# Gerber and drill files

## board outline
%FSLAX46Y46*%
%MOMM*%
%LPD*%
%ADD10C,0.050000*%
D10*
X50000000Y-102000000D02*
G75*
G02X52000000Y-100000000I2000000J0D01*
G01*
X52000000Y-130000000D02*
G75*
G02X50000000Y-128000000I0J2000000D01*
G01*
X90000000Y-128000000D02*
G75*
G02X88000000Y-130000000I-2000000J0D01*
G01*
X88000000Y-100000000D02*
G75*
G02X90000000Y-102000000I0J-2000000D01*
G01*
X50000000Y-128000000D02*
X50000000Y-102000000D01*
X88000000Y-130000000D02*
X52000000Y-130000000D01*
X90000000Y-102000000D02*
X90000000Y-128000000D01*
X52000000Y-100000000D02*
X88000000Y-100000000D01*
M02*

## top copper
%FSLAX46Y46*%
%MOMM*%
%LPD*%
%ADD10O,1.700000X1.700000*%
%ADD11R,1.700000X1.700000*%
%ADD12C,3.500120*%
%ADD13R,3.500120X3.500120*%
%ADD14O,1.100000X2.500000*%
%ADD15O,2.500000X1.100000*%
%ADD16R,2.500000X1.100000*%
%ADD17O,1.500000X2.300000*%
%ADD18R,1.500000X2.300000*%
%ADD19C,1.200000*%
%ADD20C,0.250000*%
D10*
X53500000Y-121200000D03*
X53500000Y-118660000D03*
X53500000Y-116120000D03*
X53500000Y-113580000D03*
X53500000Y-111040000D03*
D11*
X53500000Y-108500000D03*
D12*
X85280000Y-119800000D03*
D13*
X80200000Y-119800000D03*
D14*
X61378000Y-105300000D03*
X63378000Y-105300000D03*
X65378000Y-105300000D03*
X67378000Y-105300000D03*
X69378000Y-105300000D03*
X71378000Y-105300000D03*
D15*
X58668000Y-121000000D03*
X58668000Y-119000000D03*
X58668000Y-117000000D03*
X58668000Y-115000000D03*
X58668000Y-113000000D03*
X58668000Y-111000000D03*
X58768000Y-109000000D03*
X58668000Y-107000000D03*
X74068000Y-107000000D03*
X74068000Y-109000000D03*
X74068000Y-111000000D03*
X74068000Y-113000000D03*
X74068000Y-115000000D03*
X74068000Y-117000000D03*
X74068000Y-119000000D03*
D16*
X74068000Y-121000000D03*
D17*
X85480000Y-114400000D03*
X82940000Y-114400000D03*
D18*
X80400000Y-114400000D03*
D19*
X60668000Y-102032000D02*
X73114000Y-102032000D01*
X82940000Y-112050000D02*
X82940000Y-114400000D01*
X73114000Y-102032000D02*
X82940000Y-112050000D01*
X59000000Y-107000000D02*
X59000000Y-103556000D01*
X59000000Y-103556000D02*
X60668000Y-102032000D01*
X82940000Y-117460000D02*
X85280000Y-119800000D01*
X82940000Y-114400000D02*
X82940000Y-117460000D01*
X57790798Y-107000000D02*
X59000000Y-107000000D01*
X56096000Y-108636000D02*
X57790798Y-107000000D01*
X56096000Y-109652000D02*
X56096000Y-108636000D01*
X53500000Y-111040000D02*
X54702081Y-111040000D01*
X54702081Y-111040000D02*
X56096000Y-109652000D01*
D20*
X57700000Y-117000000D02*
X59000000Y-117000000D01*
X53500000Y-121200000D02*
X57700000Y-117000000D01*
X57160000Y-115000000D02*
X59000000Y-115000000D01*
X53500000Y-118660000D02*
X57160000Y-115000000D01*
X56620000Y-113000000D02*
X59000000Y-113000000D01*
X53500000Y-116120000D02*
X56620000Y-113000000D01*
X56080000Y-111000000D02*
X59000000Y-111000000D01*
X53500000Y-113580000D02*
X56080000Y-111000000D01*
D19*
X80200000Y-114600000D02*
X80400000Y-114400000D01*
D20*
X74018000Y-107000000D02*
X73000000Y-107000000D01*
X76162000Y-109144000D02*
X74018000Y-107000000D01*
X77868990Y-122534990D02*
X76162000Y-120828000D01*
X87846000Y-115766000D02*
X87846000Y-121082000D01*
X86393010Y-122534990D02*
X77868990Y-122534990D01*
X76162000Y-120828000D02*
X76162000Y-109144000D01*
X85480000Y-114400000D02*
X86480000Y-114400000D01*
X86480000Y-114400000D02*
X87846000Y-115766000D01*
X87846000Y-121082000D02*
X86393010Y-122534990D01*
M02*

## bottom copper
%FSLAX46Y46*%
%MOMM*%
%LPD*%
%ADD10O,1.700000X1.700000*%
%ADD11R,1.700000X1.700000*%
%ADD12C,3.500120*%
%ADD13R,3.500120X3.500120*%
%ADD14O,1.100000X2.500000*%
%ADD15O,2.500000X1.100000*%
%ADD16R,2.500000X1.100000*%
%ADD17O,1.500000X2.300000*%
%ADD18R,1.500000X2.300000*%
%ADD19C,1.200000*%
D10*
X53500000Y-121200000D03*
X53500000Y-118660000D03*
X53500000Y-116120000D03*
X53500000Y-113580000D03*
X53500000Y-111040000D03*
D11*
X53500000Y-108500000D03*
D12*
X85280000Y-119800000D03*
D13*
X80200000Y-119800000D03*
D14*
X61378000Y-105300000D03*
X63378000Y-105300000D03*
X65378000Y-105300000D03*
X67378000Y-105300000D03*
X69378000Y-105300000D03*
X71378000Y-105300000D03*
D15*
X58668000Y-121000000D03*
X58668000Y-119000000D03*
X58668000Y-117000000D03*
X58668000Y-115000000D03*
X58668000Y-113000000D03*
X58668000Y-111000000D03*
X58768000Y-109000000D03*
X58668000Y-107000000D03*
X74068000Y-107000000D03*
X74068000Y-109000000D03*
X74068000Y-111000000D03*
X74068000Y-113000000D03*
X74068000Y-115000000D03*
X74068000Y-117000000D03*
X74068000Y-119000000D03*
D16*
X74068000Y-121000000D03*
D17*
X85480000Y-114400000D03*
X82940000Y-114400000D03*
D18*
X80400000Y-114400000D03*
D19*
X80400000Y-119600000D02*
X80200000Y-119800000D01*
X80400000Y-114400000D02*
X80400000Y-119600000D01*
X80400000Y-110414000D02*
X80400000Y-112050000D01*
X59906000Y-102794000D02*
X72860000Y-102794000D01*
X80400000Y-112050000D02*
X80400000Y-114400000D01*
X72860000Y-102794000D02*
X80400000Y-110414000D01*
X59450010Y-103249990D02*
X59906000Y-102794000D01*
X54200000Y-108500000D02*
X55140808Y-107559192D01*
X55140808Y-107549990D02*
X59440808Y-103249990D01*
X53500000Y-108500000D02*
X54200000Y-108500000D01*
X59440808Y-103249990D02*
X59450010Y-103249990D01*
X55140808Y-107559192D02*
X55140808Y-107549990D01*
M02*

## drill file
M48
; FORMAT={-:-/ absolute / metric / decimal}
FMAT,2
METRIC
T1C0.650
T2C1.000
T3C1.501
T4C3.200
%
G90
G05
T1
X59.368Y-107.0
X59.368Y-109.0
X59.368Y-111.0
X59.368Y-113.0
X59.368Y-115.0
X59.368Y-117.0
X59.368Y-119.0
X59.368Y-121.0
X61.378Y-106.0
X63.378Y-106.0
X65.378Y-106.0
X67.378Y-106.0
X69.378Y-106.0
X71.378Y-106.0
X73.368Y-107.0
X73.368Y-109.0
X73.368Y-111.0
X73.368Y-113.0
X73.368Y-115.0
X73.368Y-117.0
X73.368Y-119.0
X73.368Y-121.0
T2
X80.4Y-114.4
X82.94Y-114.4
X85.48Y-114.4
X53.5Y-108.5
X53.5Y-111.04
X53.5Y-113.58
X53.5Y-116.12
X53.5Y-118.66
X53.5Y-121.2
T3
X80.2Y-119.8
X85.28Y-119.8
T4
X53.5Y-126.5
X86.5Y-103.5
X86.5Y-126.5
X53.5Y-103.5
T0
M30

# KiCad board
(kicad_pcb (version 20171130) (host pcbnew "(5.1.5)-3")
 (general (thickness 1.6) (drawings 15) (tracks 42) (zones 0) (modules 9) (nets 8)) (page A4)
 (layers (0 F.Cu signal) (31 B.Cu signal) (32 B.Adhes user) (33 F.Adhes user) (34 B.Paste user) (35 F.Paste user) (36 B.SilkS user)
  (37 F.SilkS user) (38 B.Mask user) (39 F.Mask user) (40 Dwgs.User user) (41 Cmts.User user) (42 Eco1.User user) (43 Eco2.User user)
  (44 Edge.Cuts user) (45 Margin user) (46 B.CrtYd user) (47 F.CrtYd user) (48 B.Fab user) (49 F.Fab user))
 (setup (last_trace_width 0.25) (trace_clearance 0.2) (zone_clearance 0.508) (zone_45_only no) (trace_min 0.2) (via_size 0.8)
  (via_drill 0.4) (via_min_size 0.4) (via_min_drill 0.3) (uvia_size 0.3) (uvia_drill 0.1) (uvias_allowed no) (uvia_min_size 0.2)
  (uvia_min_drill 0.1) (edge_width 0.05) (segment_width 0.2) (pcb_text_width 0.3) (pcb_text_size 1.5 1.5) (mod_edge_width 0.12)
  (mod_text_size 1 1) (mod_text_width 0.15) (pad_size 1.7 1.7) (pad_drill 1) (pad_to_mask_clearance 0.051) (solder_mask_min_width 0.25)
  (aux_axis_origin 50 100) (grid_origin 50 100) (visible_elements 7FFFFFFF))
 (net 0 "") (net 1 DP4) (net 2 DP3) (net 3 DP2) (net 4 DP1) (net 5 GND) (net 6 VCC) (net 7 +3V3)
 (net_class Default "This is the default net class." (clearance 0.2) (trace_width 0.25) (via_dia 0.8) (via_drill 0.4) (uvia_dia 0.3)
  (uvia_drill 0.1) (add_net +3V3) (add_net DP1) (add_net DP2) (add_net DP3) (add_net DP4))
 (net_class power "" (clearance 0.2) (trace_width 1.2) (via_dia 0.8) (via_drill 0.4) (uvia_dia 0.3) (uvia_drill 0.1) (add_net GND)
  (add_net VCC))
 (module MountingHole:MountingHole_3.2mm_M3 (layer F.Cu) (at 53.5 103.5)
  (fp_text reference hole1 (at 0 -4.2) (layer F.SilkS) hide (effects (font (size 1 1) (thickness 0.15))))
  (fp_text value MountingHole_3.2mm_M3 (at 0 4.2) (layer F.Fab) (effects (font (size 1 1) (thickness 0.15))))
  (pad 1 np_thru_hole circle (at 0 0) (size 3.2 3.2) (drill 3.2) (layers *.Cu *.Mask)))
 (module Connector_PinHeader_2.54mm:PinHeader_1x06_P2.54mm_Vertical (layer F.Cu) (at 53.5 108.5)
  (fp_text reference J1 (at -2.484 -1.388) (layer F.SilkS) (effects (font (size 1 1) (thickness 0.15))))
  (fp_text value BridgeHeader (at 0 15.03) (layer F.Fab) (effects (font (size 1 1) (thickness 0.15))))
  (pad 6 thru_hole oval (at 0 12.7) (size 1.7 1.7) (drill 1) (layers *.Cu *.Mask) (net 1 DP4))
  (pad 5 thru_hole oval (at 0 10.16) (size 1.7 1.7) (drill 1) (layers *.Cu *.Mask) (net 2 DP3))
  (pad 4 thru_hole oval (at 0 7.62) (size 1.7 1.7) (drill 1) (layers *.Cu *.Mask) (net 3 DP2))
  (pad 3 thru_hole oval (at 0 5.08) (size 1.7 1.7) (drill 1) (layers *.Cu *.Mask) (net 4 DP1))
  (pad 2 thru_hole oval (at 0 2.54) (size 1.7 1.7) (drill 1) (layers *.Cu *.Mask) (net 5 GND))
  (pad 1 thru_hole rect (at 0 0) (size 1.7 1.7) (drill 1) (layers *.Cu *.Mask) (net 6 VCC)))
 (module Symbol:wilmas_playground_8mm (layer F.Cu) (at 79.464 125.908)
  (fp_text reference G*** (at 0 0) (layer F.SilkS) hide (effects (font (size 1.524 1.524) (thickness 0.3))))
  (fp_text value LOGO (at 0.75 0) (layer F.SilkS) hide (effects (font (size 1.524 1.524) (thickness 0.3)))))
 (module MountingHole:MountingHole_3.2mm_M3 (layer F.Cu) (at 86.5 126.5)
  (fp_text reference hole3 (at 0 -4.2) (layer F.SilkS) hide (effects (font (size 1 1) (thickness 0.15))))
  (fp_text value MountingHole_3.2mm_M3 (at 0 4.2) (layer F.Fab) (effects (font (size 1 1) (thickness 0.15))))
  (pad 1 np_thru_hole circle (at 0 0) (size 3.2 3.2) (drill 3.2) (layers *.Cu *.Mask)))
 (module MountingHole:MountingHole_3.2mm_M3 (layer F.Cu) (at 86.5 103.5)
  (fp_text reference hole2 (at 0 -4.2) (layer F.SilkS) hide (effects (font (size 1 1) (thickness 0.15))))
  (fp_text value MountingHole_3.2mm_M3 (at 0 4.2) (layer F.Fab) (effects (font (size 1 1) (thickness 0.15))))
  (pad 1 np_thru_hole circle (at 0 0) (size 3.2 3.2) (drill 3.2) (layers *.Cu *.Mask)))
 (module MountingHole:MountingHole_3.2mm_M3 (layer F.Cu) (at 53.5 126.5)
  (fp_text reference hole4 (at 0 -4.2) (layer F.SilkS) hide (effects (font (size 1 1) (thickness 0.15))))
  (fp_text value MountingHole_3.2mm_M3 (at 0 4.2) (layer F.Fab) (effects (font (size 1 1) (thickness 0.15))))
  (pad 1 np_thru_hole circle (at 0 0) (size 3.2 3.2) (drill 3.2) (layers *.Cu *.Mask)))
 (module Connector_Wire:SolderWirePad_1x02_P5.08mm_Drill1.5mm (layer F.Cu) (at 80.2 119.8)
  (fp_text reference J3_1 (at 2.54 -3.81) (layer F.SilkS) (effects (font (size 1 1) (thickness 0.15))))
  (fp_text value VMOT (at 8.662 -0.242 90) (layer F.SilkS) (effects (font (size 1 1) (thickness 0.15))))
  (pad 2 thru_hole circle (at 5.08 0) (size 3.50012 3.50012) (drill 1.50114) (layers *.Cu *.Mask) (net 5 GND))
  (pad 1 thru_hole rect (at 0 0) (size 3.50012 3.50012) (drill 1.50114) (layers *.Cu *.Mask) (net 6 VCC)))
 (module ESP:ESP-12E (layer F.Cu) (at 73.368 121 180)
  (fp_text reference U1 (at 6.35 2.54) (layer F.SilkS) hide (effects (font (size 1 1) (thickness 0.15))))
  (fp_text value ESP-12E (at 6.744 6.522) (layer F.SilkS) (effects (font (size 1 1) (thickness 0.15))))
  (pad 22 thru_hole oval (at 11.99 15 270) (size 2.5 1.1) (drill 0.65 (offset -0.7 0)) (layers *.Cu *.Mask F.SilkS))
  (pad 21 thru_hole oval (at 9.99 15 270) (size 2.5 1.1) (drill 0.65 (offset -0.7 0)) (layers *.Cu *.Mask F.SilkS))
  (pad 20 thru_hole oval (at 7.99 15 270) (size 2.5 1.1) (drill 0.65 (offset -0.7 0)) (layers *.Cu *.Mask F.SilkS))
  (pad 19 thru_hole oval (at 5.99 15 270) (size 2.5 1.1) (drill 0.65 (offset -0.7 0)) (layers *.Cu *.Mask F.SilkS))
  (pad 18 thru_hole oval (at 3.99 15 270) (size 2.5 1.1) (drill 0.65 (offset -0.7 0)) (layers *.Cu *.Mask F.SilkS))
  (pad 17 thru_hole oval (at 1.99 15 270) (size 2.5 1.1) (drill 0.65 (offset -0.7 0)) (layers *.Cu *.Mask F.SilkS))
  (pad 16 thru_hole oval (at 14 0 180) (size 2.5 1.1) (drill 0.65 (offset 0.7 0)) (layers *.Cu *.Mask F.SilkS))
  (pad 15 thru_hole oval (at 14 2 180) (size 2.5 1.1) (drill 0.65 (offset 0.7 0)) (layers *.Cu *.Mask F.SilkS))
  (pad 14 thru_hole oval (at 14 4 180) (size 2.5 1.1) (drill 0.65 (offset 0.7 0)) (layers *.Cu *.Mask F.SilkS) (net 1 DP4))
  (pad 13 thru_hole oval (at 14 6 180) (size 2.5 1.1) (drill 0.65 (offset 0.7 0)) (layers *.Cu *.Mask F.SilkS) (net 2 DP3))
  (pad 12 thru_hole oval (at 14 8 180) (size 2.5 1.1) (drill 0.65 (offset 0.7 0)) (layers *.Cu *.Mask F.SilkS) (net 3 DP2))
  (pad 11 thru_hole oval (at 14 10 180) (size 2.5 1.1) (drill 0.65 (offset 0.7 0)) (layers *.Cu *.Mask F.SilkS) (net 4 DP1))
  (pad 10 thru_hole oval (at 14 12 180) (size 2.5 1.1) (drill 0.65 (offset 0.6 0)) (layers *.Cu *.Mask F.SilkS))
  (pad 9 thru_hole oval (at 14 14 180) (size 2.5 1.1) (drill 0.65 (offset 0.7 0)) (layers *.Cu *.Mask F.SilkS) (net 5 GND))
  (pad 8 thru_hole oval (at 0 14 180) (size 2.5 1.1) (drill 0.65 (offset -0.7 0)) (layers *.Cu *.Mask F.SilkS) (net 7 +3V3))
  (pad 7 thru_hole oval (at 0 12 180) (size 2.5 1.1) (drill 0.65 (offset -0.7 0)) (layers *.Cu *.Mask F.SilkS))
  (pad 6 thru_hole oval (at 0 10 180) (size 2.5 1.1) (drill 0.65 (offset -0.7 0)) (layers *.Cu *.Mask F.SilkS))
  (pad 5 thru_hole oval (at 0 8 180) (size 2.5 1.1) (drill 0.65 (offset -0.7 0)) (layers *.Cu *.Mask F.SilkS))
  (pad 4 thru_hole oval (at 0 6 180) (size 2.5 1.1) (drill 0.65 (offset -0.7 0)) (layers *.Cu *.Mask F.SilkS))
  (pad 3 thru_hole oval (at 0 4 180) (size 2.5 1.1) (drill 0.65 (offset -0.7 0)) (layers *.Cu *.Mask F.SilkS))
  (pad 2 thru_hole oval (at 0 2 180) (size 2.5 1.1) (drill 0.65 (offset -0.7 0)) (layers *.Cu *.Mask F.SilkS))
  (pad 1 thru_hole rect (at 0 0 180) (size 2.5 1.1) (drill 0.65 (offset -0.7 0)) (layers *.Cu *.Mask F.SilkS)))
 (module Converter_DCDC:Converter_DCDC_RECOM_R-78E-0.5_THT (layer F.Cu) (at 80.4 114.4)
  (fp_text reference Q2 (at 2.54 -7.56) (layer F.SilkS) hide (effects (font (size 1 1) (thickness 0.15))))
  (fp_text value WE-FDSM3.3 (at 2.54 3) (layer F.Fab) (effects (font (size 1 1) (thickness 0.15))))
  (pad 3 thru_hole oval (at 5.08 0) (size 1.5 2.3) (drill 1) (layers *.Cu *.Mask) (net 7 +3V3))
  (pad 2 thru_hole oval (at 2.54 0) (size 1.5 2.3) (drill 1) (layers *.Cu *.Mask) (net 5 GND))
  (pad 1 thru_hole rect (at 0 0) (size 1.5 2.3) (drill 1) (layers *.Cu *.Mask) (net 6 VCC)))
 (gr_arc (start 52 102) (end 52 100) (angle -90) (layer Edge.Cuts) (width 0.05))
 (gr_arc (start 52 128) (end 50 128) (angle -90) (layer Edge.Cuts) (width 0.05))
 (gr_arc (start 88 128) (end 88 130) (angle -90) (layer Edge.Cuts) (width 0.05))
 (gr_arc (start 88 102) (end 90 102) (angle -90) (layer Edge.Cuts) (width 0.05))
 (gr_line (start 50 128) (end 50 102) (layer Edge.Cuts) (width 0.05))
 (gr_line (start 88 130) (end 52 130) (layer Edge.Cuts) (width 0.05))
 (gr_line (start 90 102) (end 90 128) (layer Edge.Cuts) (width 0.05))
 (gr_line (start 52 100) (end 88 100) (layer Edge.Cuts) (width 0.05))
 (segment (start 60.668 102.032) (end 73.114 102.032) (width 1.2) (layer F.Cu) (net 5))
 (segment (start 82.94 112.05) (end 82.94 114.4) (width 1.2) (layer F.Cu) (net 5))
 (segment (start 73.114 102.032) (end 82.94 112.05) (width 1.2) (layer F.Cu) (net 5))
 (segment (start 59 107) (end 59 103.556) (width 1.2) (layer F.Cu) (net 5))
 (segment (start 59 103.556) (end 60.668 102.032) (width 1.2) (layer F.Cu) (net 5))
 (segment (start 82.94 117.46) (end 85.28 119.8) (width 1.2) (layer F.Cu) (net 5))
 (segment (start 82.94 114.4) (end 82.94 117.46) (width 1.2) (layer F.Cu) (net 5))
 (segment (start 57.790798 107) (end 59 107) (width 1.2) (layer F.Cu) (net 5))
 (segment (start 56.096 108.636) (end 57.790798 107) (width 1.2) (layer F.Cu) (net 5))
 (segment (start 56.096 109.652) (end 56.096 108.636) (width 1.2) (layer F.Cu) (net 5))
 (segment (start 53.5 111.04) (end 54.702081 111.04) (width 1.2) (layer F.Cu) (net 5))
 (segment (start 54.702081 111.04) (end 56.096 109.652) (width 1.2) (layer F.Cu) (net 5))
 (segment (start 57.7 117) (end 59 117) (width 0.25) (layer F.Cu) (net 1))
 (segment (start 53.5 121.2) (end 57.7 117) (width 0.25) (layer F.Cu) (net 1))
 (segment (start 57.16 115) (end 59 115) (width 0.25) (layer F.Cu) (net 2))
 (segment (start 53.5 118.66) (end 57.16 115) (width 0.25) (layer F.Cu) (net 2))
 (segment (start 56.62 113) (end 59 113) (width 0.25) (layer F.Cu) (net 3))
 (segment (start 53.5 116.12) (end 56.62 113) (width 0.25) (layer F.Cu) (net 3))
 (segment (start 56.08 111) (end 59 111) (width 0.25) (layer F.Cu) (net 4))
 (segment (start 53.5 113.58) (end 56.08 111) (width 0.25) (layer F.Cu) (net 4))
 (segment (start 80.2 114.6) (end 80.4 114.4) (width 1.2) (layer F.Cu) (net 6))
 (segment (start 80.4 119.6) (end 80.2 119.8) (width 1.2) (layer B.Cu) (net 6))
 (segment (start 80.4 114.4) (end 80.4 119.6) (width 1.2) (layer B.Cu) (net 6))
 (segment (start 80.4 110.414) (end 80.4 112.05) (width 1.2) (layer B.Cu) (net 6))
 (segment (start 59.906 102.794) (end 72.86 102.794) (width 1.2) (layer B.Cu) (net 6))
 (segment (start 80.4 112.05) (end 80.4 114.4) (width 1.2) (layer B.Cu) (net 6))
 (segment (start 72.86 102.794) (end 80.4 110.414) (width 1.2) (layer B.Cu) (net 6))
 (segment (start 59.45001 103.24999) (end 59.906 102.794) (width 1.2) (layer B.Cu) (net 6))
 (segment (start 54.2 108.5) (end 55.140808 107.559192) (width 1.2) (layer B.Cu) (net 6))
 (segment (start 55.140808 107.54999) (end 59.440808 103.24999) (width 1.2) (layer B.Cu) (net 6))
 (segment (start 53.5 108.5) (end 54.2 108.5) (width 1.2) (layer B.Cu) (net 6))
 (segment (start 59.440808 103.24999) (end 59.45001 103.24999) (width 1.2) (layer B.Cu) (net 6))
 (segment (start 55.140808 107.559192) (end 55.140808 107.54999) (width 1.2) (layer B.Cu) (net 6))
 (segment (start 74.018 107) (end 73 107) (width 0.25) (layer F.Cu) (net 7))
 (segment (start 76.162 109.144) (end 74.018 107) (width 0.25) (layer F.Cu) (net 7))
 (segment (start 77.86899 122.53499) (end 76.162 120.828) (width 0.25) (layer F.Cu) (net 7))
 (segment (start 87.846 115.766) (end 87.846 121.082) (width 0.25) (layer F.Cu) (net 7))
 (segment (start 86.39301 122.53499) (end 77.86899 122.53499) (width 0.25) (layer F.Cu) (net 7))
 (segment (start 76.162 120.828) (end 76.162 109.144) (width 0.25) (layer F.Cu) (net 7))
 (segment (start 85.48 114.4) (end 86.48 114.4) (width 0.25) (layer F.Cu) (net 7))
 (segment (start 86.48 114.4) (end 87.846 115.766) (width 0.25) (layer F.Cu) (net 7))
 (segment (start 87.846 121.082) (end 86.39301 122.53499) (width 0.25) (layer F.Cu) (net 7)))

